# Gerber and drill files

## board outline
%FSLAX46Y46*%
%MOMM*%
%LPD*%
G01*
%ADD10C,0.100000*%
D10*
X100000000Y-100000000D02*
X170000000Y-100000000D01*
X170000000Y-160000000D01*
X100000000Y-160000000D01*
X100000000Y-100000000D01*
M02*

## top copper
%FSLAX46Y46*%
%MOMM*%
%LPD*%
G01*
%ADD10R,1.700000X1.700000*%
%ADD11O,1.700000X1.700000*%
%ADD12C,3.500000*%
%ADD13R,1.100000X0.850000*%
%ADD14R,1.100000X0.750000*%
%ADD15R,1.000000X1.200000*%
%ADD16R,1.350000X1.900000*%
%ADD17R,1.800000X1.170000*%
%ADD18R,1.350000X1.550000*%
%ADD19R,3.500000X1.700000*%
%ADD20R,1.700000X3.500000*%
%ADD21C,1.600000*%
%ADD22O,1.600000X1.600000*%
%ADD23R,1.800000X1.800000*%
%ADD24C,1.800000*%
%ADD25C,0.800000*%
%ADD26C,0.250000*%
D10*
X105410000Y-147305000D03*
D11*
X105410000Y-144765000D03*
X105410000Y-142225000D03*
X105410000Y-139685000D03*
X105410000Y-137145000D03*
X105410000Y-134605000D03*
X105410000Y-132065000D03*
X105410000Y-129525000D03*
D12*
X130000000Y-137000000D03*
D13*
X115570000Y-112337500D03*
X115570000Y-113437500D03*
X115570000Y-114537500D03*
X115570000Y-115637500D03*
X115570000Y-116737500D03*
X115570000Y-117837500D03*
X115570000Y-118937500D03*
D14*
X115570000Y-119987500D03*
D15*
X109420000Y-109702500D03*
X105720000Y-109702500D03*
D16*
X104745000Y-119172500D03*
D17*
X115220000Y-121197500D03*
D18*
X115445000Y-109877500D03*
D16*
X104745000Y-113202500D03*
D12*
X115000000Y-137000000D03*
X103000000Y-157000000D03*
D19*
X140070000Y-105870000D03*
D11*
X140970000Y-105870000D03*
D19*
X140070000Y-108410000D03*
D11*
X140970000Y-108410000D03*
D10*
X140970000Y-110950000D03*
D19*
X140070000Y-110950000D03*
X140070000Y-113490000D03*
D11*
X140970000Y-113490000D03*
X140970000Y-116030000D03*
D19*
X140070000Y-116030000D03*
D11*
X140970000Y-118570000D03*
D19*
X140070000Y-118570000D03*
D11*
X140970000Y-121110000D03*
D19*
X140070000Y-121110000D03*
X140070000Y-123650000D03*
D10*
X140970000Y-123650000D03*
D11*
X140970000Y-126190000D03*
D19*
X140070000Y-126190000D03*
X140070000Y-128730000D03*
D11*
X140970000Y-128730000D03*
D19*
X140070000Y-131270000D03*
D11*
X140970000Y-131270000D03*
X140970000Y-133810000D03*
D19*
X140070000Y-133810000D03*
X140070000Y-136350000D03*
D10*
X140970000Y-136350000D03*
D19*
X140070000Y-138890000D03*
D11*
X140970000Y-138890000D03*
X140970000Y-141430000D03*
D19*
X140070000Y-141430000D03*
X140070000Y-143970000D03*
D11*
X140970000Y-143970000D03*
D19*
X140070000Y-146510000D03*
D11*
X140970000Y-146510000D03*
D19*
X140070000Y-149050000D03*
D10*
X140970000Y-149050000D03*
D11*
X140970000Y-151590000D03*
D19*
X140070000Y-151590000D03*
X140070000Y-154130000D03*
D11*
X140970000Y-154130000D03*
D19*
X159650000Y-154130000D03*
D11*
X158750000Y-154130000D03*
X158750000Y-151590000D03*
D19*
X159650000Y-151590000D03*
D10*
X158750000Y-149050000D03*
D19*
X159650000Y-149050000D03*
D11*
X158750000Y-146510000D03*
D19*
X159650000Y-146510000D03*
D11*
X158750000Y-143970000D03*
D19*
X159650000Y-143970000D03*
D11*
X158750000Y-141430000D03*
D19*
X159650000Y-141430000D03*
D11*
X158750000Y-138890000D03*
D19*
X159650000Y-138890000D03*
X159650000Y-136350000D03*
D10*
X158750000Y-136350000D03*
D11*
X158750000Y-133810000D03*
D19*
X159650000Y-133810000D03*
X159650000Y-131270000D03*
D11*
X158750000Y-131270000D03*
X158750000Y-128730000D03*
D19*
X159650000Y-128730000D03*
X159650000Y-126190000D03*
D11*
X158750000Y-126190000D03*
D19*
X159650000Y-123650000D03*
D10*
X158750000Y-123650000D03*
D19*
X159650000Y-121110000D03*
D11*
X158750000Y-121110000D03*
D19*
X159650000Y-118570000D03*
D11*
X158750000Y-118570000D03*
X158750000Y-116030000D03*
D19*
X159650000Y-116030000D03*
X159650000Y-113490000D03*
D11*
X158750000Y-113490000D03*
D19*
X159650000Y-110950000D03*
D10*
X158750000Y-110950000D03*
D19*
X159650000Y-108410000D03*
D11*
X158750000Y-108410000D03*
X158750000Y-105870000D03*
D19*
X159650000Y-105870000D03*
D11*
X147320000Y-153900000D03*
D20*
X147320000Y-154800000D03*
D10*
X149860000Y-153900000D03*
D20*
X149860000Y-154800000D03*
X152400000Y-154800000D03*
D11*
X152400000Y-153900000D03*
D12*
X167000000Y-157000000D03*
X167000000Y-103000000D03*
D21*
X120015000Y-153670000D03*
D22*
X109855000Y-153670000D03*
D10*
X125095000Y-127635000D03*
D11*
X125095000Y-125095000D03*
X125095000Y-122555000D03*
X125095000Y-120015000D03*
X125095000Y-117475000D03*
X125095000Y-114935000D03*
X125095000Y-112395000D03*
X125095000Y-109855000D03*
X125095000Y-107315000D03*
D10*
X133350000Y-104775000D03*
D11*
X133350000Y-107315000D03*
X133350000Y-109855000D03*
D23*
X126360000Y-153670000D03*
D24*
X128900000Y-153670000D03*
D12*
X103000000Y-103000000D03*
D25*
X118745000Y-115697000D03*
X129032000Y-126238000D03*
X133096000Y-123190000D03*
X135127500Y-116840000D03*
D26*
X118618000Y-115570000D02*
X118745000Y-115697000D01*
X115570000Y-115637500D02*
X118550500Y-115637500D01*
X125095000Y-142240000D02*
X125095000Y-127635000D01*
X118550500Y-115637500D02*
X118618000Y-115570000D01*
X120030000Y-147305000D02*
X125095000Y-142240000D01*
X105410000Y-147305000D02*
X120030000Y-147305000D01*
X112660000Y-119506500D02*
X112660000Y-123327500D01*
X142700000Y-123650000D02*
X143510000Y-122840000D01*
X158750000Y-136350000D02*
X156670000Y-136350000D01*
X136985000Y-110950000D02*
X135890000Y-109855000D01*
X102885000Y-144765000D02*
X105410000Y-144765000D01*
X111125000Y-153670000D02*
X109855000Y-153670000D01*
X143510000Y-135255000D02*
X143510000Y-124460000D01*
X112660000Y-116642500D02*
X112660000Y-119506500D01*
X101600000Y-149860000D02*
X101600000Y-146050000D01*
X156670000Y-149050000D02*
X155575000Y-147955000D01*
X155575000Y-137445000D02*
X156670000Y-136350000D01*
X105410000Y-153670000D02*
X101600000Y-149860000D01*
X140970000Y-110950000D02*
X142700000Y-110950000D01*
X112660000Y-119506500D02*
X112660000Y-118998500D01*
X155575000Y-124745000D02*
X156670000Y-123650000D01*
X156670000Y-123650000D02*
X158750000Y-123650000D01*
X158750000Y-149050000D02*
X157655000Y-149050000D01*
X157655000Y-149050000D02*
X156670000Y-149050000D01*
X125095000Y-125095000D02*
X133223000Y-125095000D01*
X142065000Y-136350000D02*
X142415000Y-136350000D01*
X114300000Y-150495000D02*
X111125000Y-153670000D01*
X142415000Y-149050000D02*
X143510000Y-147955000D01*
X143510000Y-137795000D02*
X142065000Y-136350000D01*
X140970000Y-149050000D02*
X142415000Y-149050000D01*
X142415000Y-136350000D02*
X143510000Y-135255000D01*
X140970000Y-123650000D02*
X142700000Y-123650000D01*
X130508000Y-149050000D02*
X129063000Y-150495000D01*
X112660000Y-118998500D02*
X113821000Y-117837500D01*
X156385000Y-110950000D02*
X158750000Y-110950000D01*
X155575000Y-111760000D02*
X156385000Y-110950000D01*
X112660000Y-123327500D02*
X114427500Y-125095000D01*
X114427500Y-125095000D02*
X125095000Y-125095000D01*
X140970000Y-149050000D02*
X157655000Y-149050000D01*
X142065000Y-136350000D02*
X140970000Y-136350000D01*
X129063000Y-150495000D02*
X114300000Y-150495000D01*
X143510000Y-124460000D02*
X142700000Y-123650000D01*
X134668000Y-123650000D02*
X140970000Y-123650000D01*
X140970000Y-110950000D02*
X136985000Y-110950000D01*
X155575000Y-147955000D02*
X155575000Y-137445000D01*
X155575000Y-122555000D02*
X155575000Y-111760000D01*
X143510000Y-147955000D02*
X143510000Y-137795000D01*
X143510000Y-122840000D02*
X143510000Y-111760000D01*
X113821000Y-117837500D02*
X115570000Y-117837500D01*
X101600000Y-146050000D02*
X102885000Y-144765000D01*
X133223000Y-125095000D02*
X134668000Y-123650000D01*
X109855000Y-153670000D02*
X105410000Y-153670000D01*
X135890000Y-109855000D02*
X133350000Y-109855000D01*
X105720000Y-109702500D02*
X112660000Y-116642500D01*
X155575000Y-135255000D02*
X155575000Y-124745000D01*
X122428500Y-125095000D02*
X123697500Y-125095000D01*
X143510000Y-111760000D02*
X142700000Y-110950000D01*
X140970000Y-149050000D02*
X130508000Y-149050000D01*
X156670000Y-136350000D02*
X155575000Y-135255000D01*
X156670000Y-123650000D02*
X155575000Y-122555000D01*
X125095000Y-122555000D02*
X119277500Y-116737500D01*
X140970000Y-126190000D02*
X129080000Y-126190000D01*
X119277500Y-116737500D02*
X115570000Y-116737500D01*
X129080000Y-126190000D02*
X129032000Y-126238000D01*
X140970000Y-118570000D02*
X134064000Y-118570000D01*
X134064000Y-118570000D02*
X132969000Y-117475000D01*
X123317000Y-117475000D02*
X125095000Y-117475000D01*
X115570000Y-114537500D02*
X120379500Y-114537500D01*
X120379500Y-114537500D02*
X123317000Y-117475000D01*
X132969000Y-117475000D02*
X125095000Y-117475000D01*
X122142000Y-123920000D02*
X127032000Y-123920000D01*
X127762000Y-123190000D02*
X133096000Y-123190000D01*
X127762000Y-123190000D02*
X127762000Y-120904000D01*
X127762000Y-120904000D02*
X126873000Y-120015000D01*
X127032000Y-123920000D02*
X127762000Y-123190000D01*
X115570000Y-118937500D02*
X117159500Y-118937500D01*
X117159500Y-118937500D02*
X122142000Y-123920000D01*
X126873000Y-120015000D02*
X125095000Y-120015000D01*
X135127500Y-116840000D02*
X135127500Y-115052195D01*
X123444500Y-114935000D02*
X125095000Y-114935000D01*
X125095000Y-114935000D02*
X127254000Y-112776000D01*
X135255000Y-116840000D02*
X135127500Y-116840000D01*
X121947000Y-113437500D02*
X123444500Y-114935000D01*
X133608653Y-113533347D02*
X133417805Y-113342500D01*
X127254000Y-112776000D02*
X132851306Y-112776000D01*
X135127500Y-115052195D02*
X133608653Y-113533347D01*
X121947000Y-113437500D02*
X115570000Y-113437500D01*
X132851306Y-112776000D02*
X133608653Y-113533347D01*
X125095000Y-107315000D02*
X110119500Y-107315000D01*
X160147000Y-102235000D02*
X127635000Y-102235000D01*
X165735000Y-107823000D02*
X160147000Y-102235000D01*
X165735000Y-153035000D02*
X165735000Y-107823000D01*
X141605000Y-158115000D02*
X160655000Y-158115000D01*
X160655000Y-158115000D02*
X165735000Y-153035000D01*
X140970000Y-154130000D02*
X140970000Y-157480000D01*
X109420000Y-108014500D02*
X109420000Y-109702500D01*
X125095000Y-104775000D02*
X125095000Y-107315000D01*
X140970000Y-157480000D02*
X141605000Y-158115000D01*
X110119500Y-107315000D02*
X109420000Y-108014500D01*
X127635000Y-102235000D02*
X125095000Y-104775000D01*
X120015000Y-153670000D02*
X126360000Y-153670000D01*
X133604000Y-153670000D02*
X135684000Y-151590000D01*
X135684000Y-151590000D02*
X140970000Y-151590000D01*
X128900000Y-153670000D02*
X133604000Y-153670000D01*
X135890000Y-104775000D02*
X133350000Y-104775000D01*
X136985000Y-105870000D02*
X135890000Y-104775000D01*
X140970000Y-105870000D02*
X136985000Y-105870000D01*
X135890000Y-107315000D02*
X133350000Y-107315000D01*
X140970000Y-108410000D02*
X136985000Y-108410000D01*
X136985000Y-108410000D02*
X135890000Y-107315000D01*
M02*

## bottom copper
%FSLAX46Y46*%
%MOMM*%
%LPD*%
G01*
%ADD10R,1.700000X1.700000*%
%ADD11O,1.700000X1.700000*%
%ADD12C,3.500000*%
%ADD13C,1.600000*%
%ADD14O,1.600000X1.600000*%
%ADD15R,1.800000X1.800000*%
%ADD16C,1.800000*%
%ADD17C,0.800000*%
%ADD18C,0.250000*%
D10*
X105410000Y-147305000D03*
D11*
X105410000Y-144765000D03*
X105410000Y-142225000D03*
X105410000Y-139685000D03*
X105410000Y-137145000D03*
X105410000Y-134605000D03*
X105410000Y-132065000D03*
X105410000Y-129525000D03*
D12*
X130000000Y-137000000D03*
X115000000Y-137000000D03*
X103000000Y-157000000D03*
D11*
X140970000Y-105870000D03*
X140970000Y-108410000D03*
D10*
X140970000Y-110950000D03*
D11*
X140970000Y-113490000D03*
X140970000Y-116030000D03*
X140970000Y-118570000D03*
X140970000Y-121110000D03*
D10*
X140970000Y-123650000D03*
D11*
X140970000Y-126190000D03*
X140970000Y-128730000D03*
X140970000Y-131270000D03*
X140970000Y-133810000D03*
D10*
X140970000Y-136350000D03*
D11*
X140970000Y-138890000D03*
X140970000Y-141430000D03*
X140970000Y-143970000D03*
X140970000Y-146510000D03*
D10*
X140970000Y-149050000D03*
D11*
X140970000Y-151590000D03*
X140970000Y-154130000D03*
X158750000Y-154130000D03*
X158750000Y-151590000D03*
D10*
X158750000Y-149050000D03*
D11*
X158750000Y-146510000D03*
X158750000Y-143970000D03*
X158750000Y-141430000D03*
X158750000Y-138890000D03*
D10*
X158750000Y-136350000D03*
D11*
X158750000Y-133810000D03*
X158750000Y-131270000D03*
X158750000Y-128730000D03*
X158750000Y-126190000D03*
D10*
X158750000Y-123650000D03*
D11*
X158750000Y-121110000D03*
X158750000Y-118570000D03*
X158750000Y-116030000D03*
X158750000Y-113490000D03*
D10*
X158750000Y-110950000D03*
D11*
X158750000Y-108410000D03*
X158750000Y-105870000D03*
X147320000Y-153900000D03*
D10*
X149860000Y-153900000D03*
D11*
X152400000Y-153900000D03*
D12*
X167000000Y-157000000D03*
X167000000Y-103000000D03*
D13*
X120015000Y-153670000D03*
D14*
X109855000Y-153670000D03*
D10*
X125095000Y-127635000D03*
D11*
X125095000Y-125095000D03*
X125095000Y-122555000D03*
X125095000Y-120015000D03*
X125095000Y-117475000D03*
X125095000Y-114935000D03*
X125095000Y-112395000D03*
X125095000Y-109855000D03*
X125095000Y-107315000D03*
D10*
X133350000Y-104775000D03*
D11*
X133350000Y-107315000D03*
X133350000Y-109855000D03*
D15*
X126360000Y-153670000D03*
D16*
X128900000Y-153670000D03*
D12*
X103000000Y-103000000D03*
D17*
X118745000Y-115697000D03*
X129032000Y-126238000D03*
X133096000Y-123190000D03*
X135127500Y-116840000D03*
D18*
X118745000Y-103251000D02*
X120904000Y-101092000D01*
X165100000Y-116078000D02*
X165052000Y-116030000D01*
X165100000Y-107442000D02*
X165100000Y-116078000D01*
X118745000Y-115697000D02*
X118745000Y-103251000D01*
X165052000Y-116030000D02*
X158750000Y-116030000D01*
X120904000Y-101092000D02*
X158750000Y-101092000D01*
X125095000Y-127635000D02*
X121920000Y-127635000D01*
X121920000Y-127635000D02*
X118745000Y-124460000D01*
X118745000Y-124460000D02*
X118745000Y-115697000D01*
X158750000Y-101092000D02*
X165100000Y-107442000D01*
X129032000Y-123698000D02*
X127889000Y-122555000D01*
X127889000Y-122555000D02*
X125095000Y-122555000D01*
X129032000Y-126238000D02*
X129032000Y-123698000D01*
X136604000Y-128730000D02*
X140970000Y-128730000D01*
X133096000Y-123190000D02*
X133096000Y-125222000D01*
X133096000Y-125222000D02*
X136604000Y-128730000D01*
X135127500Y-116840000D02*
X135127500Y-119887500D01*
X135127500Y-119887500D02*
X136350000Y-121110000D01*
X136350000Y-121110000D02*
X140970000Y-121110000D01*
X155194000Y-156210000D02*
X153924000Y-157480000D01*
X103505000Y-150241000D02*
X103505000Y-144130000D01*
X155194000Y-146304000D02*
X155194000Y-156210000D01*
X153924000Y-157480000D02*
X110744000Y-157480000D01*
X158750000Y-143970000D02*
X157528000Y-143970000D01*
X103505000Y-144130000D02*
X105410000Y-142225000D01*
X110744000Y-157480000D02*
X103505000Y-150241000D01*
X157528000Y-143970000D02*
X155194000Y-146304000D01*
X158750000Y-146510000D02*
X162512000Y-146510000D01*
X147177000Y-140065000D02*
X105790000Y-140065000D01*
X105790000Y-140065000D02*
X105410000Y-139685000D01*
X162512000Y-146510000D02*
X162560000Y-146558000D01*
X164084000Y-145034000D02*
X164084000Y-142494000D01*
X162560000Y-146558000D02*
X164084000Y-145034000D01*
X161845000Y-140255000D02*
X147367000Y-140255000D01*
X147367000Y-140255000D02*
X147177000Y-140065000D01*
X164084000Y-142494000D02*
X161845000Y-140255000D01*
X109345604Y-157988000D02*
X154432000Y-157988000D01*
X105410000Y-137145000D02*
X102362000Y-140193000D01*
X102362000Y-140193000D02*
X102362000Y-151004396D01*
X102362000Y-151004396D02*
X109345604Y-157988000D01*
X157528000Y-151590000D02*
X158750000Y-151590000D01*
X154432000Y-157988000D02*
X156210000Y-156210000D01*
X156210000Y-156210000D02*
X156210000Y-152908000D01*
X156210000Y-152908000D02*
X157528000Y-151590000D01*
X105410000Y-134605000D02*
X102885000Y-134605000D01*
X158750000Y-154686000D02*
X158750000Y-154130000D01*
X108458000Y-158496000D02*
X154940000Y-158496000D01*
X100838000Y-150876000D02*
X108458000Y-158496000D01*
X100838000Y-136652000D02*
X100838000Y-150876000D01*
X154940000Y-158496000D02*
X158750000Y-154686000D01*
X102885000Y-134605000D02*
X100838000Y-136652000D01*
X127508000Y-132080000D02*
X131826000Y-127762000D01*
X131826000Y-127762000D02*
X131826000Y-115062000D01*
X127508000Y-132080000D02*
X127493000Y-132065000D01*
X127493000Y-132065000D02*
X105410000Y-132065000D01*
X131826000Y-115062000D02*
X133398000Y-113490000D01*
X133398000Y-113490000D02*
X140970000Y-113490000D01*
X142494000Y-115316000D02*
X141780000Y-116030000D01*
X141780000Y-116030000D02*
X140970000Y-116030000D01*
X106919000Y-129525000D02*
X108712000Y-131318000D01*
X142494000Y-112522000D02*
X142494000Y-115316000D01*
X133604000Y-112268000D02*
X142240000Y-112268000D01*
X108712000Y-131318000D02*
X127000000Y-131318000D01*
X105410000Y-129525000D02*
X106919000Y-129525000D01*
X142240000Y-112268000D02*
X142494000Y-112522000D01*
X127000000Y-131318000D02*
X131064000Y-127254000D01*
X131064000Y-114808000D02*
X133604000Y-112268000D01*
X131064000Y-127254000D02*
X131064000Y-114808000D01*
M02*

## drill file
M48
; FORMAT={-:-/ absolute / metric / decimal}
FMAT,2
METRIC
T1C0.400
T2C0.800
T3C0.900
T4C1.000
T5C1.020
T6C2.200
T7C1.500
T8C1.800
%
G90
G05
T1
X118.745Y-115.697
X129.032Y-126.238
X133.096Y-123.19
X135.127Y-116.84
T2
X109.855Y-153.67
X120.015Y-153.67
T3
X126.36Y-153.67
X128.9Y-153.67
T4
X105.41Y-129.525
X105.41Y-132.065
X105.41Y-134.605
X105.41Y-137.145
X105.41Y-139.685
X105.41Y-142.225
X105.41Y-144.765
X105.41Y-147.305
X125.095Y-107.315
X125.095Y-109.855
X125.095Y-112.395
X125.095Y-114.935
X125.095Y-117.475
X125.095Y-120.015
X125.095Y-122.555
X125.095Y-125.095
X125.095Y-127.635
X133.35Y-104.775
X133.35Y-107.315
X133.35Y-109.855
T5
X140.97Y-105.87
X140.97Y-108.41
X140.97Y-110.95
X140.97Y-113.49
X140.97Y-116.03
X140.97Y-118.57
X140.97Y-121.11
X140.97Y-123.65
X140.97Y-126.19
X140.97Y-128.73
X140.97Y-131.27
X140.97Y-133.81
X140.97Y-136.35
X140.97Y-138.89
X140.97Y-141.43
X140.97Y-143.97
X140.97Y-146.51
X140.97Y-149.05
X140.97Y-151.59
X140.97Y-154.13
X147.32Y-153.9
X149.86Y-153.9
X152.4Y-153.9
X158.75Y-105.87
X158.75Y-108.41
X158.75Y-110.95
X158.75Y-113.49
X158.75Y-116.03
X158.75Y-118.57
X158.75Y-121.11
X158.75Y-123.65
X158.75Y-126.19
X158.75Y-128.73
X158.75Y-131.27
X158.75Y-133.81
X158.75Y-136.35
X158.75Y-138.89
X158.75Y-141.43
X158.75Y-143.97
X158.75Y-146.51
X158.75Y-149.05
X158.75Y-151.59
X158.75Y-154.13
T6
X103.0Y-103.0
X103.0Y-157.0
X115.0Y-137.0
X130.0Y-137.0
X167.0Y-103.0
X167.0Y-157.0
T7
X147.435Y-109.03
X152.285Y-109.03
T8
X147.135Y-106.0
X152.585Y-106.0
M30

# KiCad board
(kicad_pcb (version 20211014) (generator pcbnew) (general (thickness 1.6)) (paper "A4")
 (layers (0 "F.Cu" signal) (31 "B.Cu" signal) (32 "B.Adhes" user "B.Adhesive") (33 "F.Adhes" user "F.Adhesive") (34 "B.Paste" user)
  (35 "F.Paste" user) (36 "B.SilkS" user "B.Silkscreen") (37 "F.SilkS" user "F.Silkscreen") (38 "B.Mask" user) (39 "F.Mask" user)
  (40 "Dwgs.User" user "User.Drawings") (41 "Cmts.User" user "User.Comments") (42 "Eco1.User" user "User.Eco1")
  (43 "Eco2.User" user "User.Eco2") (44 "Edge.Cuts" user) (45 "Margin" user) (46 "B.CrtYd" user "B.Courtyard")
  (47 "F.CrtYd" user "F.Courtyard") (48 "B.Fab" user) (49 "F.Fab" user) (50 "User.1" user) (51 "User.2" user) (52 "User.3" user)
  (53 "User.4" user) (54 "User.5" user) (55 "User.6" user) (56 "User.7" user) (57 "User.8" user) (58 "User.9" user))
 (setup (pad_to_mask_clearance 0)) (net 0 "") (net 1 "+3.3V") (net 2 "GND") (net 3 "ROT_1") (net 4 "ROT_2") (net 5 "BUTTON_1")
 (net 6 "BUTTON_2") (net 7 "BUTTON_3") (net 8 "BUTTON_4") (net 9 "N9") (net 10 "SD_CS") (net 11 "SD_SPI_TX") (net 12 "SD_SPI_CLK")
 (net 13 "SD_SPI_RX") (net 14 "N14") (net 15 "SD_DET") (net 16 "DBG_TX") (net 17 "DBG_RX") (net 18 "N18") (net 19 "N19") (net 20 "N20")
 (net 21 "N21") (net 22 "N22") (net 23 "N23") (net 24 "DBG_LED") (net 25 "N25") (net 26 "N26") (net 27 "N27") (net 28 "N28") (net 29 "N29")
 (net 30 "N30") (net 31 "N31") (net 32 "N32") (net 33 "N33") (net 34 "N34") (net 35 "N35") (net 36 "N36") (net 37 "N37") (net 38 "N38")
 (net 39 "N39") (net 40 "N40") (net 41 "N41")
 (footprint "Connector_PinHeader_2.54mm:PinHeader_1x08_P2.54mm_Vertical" (layer "F.Cu") (at 105.41 147.305 180)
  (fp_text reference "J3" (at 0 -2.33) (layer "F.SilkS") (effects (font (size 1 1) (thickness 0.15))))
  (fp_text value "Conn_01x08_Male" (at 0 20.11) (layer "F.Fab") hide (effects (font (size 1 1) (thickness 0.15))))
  (pad "1" thru_hole rect (at 0 0 180) (size 1.7 1.7) (drill 1) (layers *.Cu *.Mask) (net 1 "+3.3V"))
  (pad "2" thru_hole oval (at 0 2.54 180) (size 1.7 1.7) (drill 1) (layers *.Cu *.Mask) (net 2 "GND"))
  (pad "3" thru_hole oval (at 0 5.08 180) (size 1.7 1.7) (drill 1) (layers *.Cu *.Mask) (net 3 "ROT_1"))
  (pad "4" thru_hole oval (at 0 7.62 180) (size 1.7 1.7) (drill 1) (layers *.Cu *.Mask) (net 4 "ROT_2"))
  (pad "5" thru_hole oval (at 0 10.16 180) (size 1.7 1.7) (drill 1) (layers *.Cu *.Mask) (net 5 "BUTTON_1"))
  (pad "6" thru_hole oval (at 0 12.7 180) (size 1.7 1.7) (drill 1) (layers *.Cu *.Mask) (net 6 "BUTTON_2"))
  (pad "7" thru_hole oval (at 0 15.24 180) (size 1.7 1.7) (drill 1) (layers *.Cu *.Mask) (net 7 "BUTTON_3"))
  (pad "8" thru_hole oval (at 0 17.78 180) (size 1.7 1.7) (drill 1) (layers *.Cu *.Mask) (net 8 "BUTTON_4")))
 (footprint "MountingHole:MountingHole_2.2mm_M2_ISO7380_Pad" (layer "F.Cu") (at 130 137)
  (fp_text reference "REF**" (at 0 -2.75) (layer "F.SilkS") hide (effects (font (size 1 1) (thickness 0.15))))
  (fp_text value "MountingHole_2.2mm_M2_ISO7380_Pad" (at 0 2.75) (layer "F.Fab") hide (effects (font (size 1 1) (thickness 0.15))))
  (pad "1" thru_hole circle (at 0 0) (size 3.5 3.5) (drill 2.2) (layers *.Cu *.Mask)))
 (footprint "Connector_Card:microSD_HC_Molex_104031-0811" (layer "F.Cu") (at 110.12 115.4425 -90)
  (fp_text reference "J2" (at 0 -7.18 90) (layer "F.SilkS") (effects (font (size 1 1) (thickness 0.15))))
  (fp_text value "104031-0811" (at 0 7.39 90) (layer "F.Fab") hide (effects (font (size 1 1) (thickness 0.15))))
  (pad "1" smd rect (at -3.105 -5.45 270) (size 0.85 1.1) (layers "F.Cu" "F.Paste" "F.Mask") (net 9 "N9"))
  (pad "2" smd rect (at -2.005 -5.45 270) (size 0.85 1.1) (layers "F.Cu" "F.Paste" "F.Mask") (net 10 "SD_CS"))
  (pad "3" smd rect (at -0.905 -5.45 270) (size 0.85 1.1) (layers "F.Cu" "F.Paste" "F.Mask") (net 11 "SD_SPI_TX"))
  (pad "4" smd rect (at 0.195 -5.45 270) (size 0.85 1.1) (layers "F.Cu" "F.Paste" "F.Mask") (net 1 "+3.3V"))
  (pad "5" smd rect (at 1.295 -5.45 270) (size 0.85 1.1) (layers "F.Cu" "F.Paste" "F.Mask") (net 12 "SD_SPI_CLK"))
  (pad "6" smd rect (at 2.395 -5.45 270) (size 0.85 1.1) (layers "F.Cu" "F.Paste" "F.Mask") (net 2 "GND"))
  (pad "7" smd rect (at 3.495 -5.45 270) (size 0.85 1.1) (layers "F.Cu" "F.Paste" "F.Mask") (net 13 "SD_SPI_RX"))
  (pad "8" smd rect (at 4.545 -5.45 270) (size 0.75 1.1) (layers "F.Cu" "F.Paste" "F.Mask") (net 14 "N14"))
  (pad "9" smd rect (at -5.74 0.7 270) (size 1.2 1) (layers "F.Cu" "F.Paste" "F.Mask") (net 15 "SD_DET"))
  (pad "10" smd rect (at -5.74 4.4 270) (size 1.2 1) (layers "F.Cu" "F.Paste" "F.Mask") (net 2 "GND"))
  (pad "11" smd rect (at 3.73 5.375 270) (size 1.9 1.35) (layers "F.Cu" "F.Paste" "F.Mask"))
  (pad "11" smd rect (at 5.755 -5.1 270) (size 1.17 1.8) (layers "F.Cu" "F.Paste" "F.Mask"))
  (pad "11" smd rect (at -5.565 -5.325 270) (size 1.55 1.35) (layers "F.Cu" "F.Paste" "F.Mask"))
  (pad "11" smd rect (at -2.24 5.375 270) (size 1.9 1.35) (layers "F.Cu" "F.Paste" "F.Mask")))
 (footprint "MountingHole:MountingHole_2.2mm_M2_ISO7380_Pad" (layer "F.Cu") (at 115 137)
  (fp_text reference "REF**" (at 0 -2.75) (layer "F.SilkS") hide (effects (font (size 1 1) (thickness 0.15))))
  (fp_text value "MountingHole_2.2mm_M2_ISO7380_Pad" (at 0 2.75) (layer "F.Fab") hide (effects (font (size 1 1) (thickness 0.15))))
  (pad "1" thru_hole circle (at 0 0) (size 3.5 3.5) (drill 2.2) (layers *.Cu *.Mask)))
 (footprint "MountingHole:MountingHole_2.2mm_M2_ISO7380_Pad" (layer "F.Cu") (at 103 157)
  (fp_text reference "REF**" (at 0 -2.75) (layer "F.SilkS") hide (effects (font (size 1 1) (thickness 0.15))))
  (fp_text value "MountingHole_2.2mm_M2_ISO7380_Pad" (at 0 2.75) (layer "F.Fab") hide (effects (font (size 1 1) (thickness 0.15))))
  (pad "1" thru_hole circle (at 0 0) (size 3.5 3.5) (drill 2.2) (layers *.Cu *.Mask)))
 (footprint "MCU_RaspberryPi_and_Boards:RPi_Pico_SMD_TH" (layer "F.Cu") (at 149.86 130)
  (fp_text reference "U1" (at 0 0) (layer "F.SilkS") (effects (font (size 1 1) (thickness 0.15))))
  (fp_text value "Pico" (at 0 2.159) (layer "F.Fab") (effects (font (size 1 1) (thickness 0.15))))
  (pad "" np_thru_hole oval (at 2.425 -20.97) (size 1.5 1.5) (drill 1.5) (layers *.Cu *.Mask))
  (pad "" np_thru_hole oval (at -2.425 -20.97) (size 1.5 1.5) (drill 1.5) (layers *.Cu *.Mask))
  (pad "" np_thru_hole oval (at -2.725 -24) (size 1.8 1.8) (drill 1.8) (layers *.Cu *.Mask))
  (pad "" np_thru_hole oval (at 2.725 -24) (size 1.8 1.8) (drill 1.8) (layers *.Cu *.Mask))
  (pad "1" smd rect (at -8.89 -24.13) (size 3.5 1.7) (drill (offset -0.9 0)) (layers "F.Cu" "F.Mask") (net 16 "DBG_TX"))
  (pad "1" thru_hole oval (at -8.89 -24.13) (size 1.7 1.7) (drill 1.02) (layers *.Cu *.Mask) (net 16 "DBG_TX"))
  (pad "2" smd rect (at -8.89 -21.59) (size 3.5 1.7) (drill (offset -0.9 0)) (layers "F.Cu" "F.Mask") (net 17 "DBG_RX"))
  (pad "2" thru_hole oval (at -8.89 -21.59) (size 1.7 1.7) (drill 1.02) (layers *.Cu *.Mask) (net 17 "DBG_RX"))
  (pad "3" thru_hole rect (at -8.89 -19.05) (size 1.7 1.7) (drill 1.02) (layers *.Cu *.Mask) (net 2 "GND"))
  (pad "3" smd rect (at -8.89 -19.05) (size 3.5 1.7) (drill (offset -0.9 0)) (layers "F.Cu" "F.Mask") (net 2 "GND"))
  (pad "4" smd rect (at -8.89 -16.51) (size 3.5 1.7) (drill (offset -0.9 0)) (layers "F.Cu" "F.Mask") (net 7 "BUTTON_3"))
  (pad "4" thru_hole oval (at -8.89 -16.51) (size 1.7 1.7) (drill 1.02) (layers *.Cu *.Mask) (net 7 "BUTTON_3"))
  (pad "5" thru_hole oval (at -8.89 -13.97) (size 1.7 1.7) (drill 1.02) (layers *.Cu *.Mask) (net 8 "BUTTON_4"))
  (pad "5" smd rect (at -8.89 -13.97) (size 3.5 1.7) (drill (offset -0.9 0)) (layers "F.Cu" "F.Mask") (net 8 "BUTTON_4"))
  (pad "6" thru_hole oval (at -8.89 -11.43) (size 1.7 1.7) (drill 1.02) (layers *.Cu *.Mask) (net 11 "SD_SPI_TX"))
  (pad "6" smd rect (at -8.89 -11.43) (size 3.5 1.7) (drill (offset -0.9 0)) (layers "F.Cu" "F.Mask") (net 11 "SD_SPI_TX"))
  (pad "7" thru_hole oval (at -8.89 -8.89) (size 1.7 1.7) (drill 1.02) (layers *.Cu *.Mask) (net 10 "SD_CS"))
  (pad "7" smd rect (at -8.89 -8.89) (size 3.5 1.7) (drill (offset -0.9 0)) (layers "F.Cu" "F.Mask") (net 10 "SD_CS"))
  (pad "8" smd rect (at -8.89 -6.35) (size 3.5 1.7) (drill (offset -0.9 0)) (layers "F.Cu" "F.Mask") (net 2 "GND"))
  (pad "8" thru_hole rect (at -8.89 -6.35) (size 1.7 1.7) (drill 1.02) (layers *.Cu *.Mask) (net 2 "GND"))
  (pad "9" thru_hole oval (at -8.89 -3.81) (size 1.7 1.7) (drill 1.02) (layers *.Cu *.Mask) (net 12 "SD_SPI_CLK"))
  (pad "9" smd rect (at -8.89 -3.81) (size 3.5 1.7) (drill (offset -0.9 0)) (layers "F.Cu" "F.Mask") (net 12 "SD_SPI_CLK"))
  (pad "10" smd rect (at -8.89 -1.27) (size 3.5 1.7) (drill (offset -0.9 0)) (layers "F.Cu" "F.Mask") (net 13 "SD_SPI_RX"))
  (pad "10" thru_hole oval (at -8.89 -1.27) (size 1.7 1.7) (drill 1.02) (layers *.Cu *.Mask) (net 13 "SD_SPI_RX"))
  (pad "11" smd rect (at -8.89 1.27) (size 3.5 1.7) (drill (offset -0.9 0)) (layers "F.Cu" "F.Mask") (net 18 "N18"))
  (pad "11" thru_hole oval (at -8.89 1.27) (size 1.7 1.7) (drill 1.02) (layers *.Cu *.Mask) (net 18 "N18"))
  (pad "12" thru_hole oval (at -8.89 3.81) (size 1.7 1.7) (drill 1.02) (layers *.Cu *.Mask) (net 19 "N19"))
  (pad "12" smd rect (at -8.89 3.81) (size 3.5 1.7) (drill (offset -0.9 0)) (layers "F.Cu" "F.Mask") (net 19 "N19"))
  (pad "13" smd rect (at -8.89 6.35) (size 3.5 1.7) (drill (offset -0.9 0)) (layers "F.Cu" "F.Mask") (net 2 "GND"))
  (pad "13" thru_hole rect (at -8.89 6.35) (size 1.7 1.7) (drill 1.02) (layers *.Cu *.Mask) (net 2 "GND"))
  (pad "14" smd rect (at -8.89 8.89) (size 3.5 1.7) (drill (offset -0.9 0)) (layers "F.Cu" "F.Mask") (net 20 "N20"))
  (pad "14" thru_hole oval (at -8.89 8.89) (size 1.7 1.7) (drill 1.02) (layers *.Cu *.Mask) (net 20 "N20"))
  (pad "15" thru_hole oval (at -8.89 11.43) (size 1.7 1.7) (drill 1.02) (layers *.Cu *.Mask) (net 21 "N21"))
  (pad "15" smd rect (at -8.89 11.43) (size 3.5 1.7) (drill (offset -0.9 0)) (layers "F.Cu" "F.Mask") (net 21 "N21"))
  (pad "16" smd rect (at -8.89 13.97) (size 3.5 1.7) (drill (offset -0.9 0)) (layers "F.Cu" "F.Mask") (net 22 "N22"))
  (pad "16" thru_hole oval (at -8.89 13.97) (size 1.7 1.7) (drill 1.02) (layers *.Cu *.Mask) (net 22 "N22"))
  (pad "17" smd rect (at -8.89 16.51) (size 3.5 1.7) (drill (offset -0.9 0)) (layers "F.Cu" "F.Mask") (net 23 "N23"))
  (pad "17" thru_hole oval (at -8.89 16.51) (size 1.7 1.7) (drill 1.02) (layers *.Cu *.Mask) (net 23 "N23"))
  (pad "18" smd rect (at -8.89 19.05) (size 3.5 1.7) (drill (offset -0.9 0)) (layers "F.Cu" "F.Mask") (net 2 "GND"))
  (pad "18" thru_hole rect (at -8.89 19.05) (size 1.7 1.7) (drill 1.02) (layers *.Cu *.Mask) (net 2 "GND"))
  (pad "19" thru_hole oval (at -8.89 21.59) (size 1.7 1.7) (drill 1.02) (layers *.Cu *.Mask) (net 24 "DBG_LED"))
  (pad "19" smd rect (at -8.89 21.59) (size 3.5 1.7) (drill (offset -0.9 0)) (layers "F.Cu" "F.Mask") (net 24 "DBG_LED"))
  (pad "20" smd rect (at -8.89 24.13) (size 3.5 1.7) (drill (offset -0.9 0)) (layers "F.Cu" "F.Mask") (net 15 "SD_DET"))
  (pad "20" thru_hole oval (at -8.89 24.13) (size 1.7 1.7) (drill 1.02) (layers *.Cu *.Mask) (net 15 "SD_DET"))
  (pad "21" smd rect (at 8.89 24.13) (size 3.5 1.7) (drill (offset 0.9 0)) (layers "F.Cu" "F.Mask") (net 6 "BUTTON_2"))
  (pad "21" thru_hole oval (at 8.89 24.13) (size 1.7 1.7) (drill 1.02) (layers *.Cu *.Mask) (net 6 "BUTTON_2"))
  (pad "22" thru_hole oval (at 8.89 21.59) (size 1.7 1.7) (drill 1.02) (layers *.Cu *.Mask) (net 5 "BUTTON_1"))
  (pad "22" smd rect (at 8.89 21.59) (size 3.5 1.7) (drill (offset 0.9 0)) (layers "F.Cu" "F.Mask") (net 5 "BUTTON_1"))
  (pad "23" thru_hole rect (at 8.89 19.05) (size 1.7 1.7) (drill 1.02) (layers *.Cu *.Mask) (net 2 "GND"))
  (pad "23" smd rect (at 8.89 19.05) (size 3.5 1.7) (drill (offset 0.9 0)) (layers "F.Cu" "F.Mask") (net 2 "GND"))
  (pad "24" thru_hole oval (at 8.89 16.51) (size 1.7 1.7) (drill 1.02) (layers *.Cu *.Mask) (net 4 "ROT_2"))
  (pad "24" smd rect (at 8.89 16.51) (size 3.5 1.7) (drill (offset 0.9 0)) (layers "F.Cu" "F.Mask") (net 4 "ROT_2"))
  (pad "25" thru_hole oval (at 8.89 13.97) (size 1.7 1.7) (drill 1.02) (layers *.Cu *.Mask) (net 3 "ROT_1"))
  (pad "25" smd rect (at 8.89 13.97) (size 3.5 1.7) (drill (offset 0.9 0)) (layers "F.Cu" "F.Mask") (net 3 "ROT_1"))
  (pad "26" thru_hole oval (at 8.89 11.43) (size 1.7 1.7) (drill 1.02) (layers *.Cu *.Mask) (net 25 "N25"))
  (pad "26" smd rect (at 8.89 11.43) (size 3.5 1.7) (drill (offset 0.9 0)) (layers "F.Cu" "F.Mask") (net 25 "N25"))
  (pad "27" thru_hole oval (at 8.89 8.89) (size 1.7 1.7) (drill 1.02) (layers *.Cu *.Mask) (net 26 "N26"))
  (pad "27" smd rect (at 8.89 8.89) (size 3.5 1.7) (drill (offset 0.9 0)) (layers "F.Cu" "F.Mask") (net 26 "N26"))
  (pad "28" smd rect (at 8.89 6.35) (size 3.5 1.7) (drill (offset 0.9 0)) (layers "F.Cu" "F.Mask") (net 2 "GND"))
  (pad "28" thru_hole rect (at 8.89 6.35) (size 1.7 1.7) (drill 1.02) (layers *.Cu *.Mask) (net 2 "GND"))
  (pad "29" thru_hole oval (at 8.89 3.81) (size 1.7 1.7) (drill 1.02) (layers *.Cu *.Mask) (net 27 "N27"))
  (pad "29" smd rect (at 8.89 3.81) (size 3.5 1.7) (drill (offset 0.9 0)) (layers "F.Cu" "F.Mask") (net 27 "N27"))
  (pad "30" smd rect (at 8.89 1.27) (size 3.5 1.7) (drill (offset 0.9 0)) (layers "F.Cu" "F.Mask") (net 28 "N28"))
  (pad "30" thru_hole oval (at 8.89 1.27) (size 1.7 1.7) (drill 1.02) (layers *.Cu *.Mask) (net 28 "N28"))
  (pad "31" thru_hole oval (at 8.89 -1.27) (size 1.7 1.7) (drill 1.02) (layers *.Cu *.Mask) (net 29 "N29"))
  (pad "31" smd rect (at 8.89 -1.27) (size 3.5 1.7) (drill (offset 0.9 0)) (layers "F.Cu" "F.Mask") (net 29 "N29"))
  (pad "32" smd rect (at 8.89 -3.81) (size 3.5 1.7) (drill (offset 0.9 0)) (layers "F.Cu" "F.Mask") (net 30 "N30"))
  (pad "32" thru_hole oval (at 8.89 -3.81) (size 1.7 1.7) (drill 1.02) (layers *.Cu *.Mask) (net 30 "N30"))
  (pad "33" smd rect (at 8.89 -6.35) (size 3.5 1.7) (drill (offset 0.9 0)) (layers "F.Cu" "F.Mask") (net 2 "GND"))
  (pad "33" thru_hole rect (at 8.89 -6.35) (size 1.7 1.7) (drill 1.02) (layers *.Cu *.Mask) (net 2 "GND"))
  (pad "34" smd rect (at 8.89 -8.89) (size 3.5 1.7) (drill (offset 0.9 0)) (layers "F.Cu" "F.Mask") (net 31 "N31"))
  (pad "34" thru_hole oval (at 8.89 -8.89) (size 1.7 1.7) (drill 1.02) (layers *.Cu *.Mask) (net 31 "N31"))
  (pad "35" smd rect (at 8.89 -11.43) (size 3.5 1.7) (drill (offset 0.9 0)) (layers "F.Cu" "F.Mask") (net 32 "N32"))
  (pad "35" thru_hole oval (at 8.89 -11.43) (size 1.7 1.7) (drill 1.02) (layers *.Cu *.Mask) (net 32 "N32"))
  (pad "36" thru_hole oval (at 8.89 -13.97) (size 1.7 1.7) (drill 1.02) (layers *.Cu *.Mask) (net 1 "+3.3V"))
  (pad "36" smd rect (at 8.89 -13.97) (size 3.5 1.7) (drill (offset 0.9 0)) (layers "F.Cu" "F.Mask") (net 1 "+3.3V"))
  (pad "37" smd rect (at 8.89 -16.51) (size 3.5 1.7) (drill (offset 0.9 0)) (layers "F.Cu" "F.Mask") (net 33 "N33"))
  (pad "37" thru_hole oval (at 8.89 -16.51) (size 1.7 1.7) (drill 1.02) (layers *.Cu *.Mask) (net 33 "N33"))
  (pad "38" smd rect (at 8.89 -19.05) (size 3.5 1.7) (drill (offset 0.9 0)) (layers "F.Cu" "F.Mask") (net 2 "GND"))
  (pad "38" thru_hole rect (at 8.89 -19.05) (size 1.7 1.7) (drill 1.02) (layers *.Cu *.Mask) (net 2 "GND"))
  (pad "39" smd rect (at 8.89 -21.59) (size 3.5 1.7) (drill (offset 0.9 0)) (layers "F.Cu" "F.Mask") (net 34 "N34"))
  (pad "39" thru_hole oval (at 8.89 -21.59) (size 1.7 1.7) (drill 1.02) (layers *.Cu *.Mask) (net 34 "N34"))
  (pad "40" thru_hole oval (at 8.89 -24.13) (size 1.7 1.7) (drill 1.02) (layers *.Cu *.Mask) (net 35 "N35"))
  (pad "40" smd rect (at 8.89 -24.13) (size 3.5 1.7) (drill (offset 0.9 0)) (layers "F.Cu" "F.Mask") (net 35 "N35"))
  (pad "41" thru_hole oval (at -2.54 23.9) (size 1.7 1.7) (drill 1.02) (layers *.Cu *.Mask) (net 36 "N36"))
  (pad "41" smd rect (at -2.54 23.9 90) (size 3.5 1.7) (drill (offset -0.9 0)) (layers "F.Cu" "F.Mask") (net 36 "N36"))
  (pad "42" thru_hole rect (at 0 23.9) (size 1.7 1.7) (drill 1.02) (layers *.Cu *.Mask) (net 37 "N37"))
  (pad "42" smd rect (at 0 23.9 90) (size 3.5 1.7) (drill (offset -0.9 0)) (layers "F.Cu" "F.Mask") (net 37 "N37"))
  (pad "43" smd rect (at 2.54 23.9 90) (size 3.5 1.7) (drill (offset -0.9 0)) (layers "F.Cu" "F.Mask") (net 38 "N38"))
  (pad "43" thru_hole oval (at 2.54 23.9) (size 1.7 1.7) (drill 1.02) (layers *.Cu *.Mask) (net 38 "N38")))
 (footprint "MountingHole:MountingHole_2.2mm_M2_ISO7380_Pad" (layer "F.Cu") (at 167 157)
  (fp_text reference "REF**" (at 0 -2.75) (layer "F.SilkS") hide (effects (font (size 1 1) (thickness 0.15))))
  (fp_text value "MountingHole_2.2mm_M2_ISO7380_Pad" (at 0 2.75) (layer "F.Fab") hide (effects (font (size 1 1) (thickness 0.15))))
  (pad "1" thru_hole circle (at 0 0) (size 3.5 3.5) (drill 2.2) (layers *.Cu *.Mask)))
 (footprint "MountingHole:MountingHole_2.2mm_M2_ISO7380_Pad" (layer "F.Cu") (at 167 103)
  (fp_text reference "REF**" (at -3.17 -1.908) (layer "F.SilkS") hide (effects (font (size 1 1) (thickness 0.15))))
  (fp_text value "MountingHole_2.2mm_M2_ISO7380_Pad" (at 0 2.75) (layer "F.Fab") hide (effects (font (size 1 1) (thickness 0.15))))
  (pad "1" thru_hole circle (at 0 0) (size 3.5 3.5) (drill 2.2) (layers *.Cu *.Mask)))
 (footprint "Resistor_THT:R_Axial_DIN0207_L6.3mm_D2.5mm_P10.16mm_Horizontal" (layer "F.Cu") (at 120.015 153.67 180)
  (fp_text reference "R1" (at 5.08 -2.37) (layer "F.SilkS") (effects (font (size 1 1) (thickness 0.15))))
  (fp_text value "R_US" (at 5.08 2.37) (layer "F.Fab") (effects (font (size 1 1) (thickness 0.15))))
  (pad "1" thru_hole circle (at 0 0 180) (size 1.6 1.6) (drill 0.8) (layers *.Cu *.Mask) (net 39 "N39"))
  (pad "2" thru_hole oval (at 10.16 0 180) (size 1.6 1.6) (drill 0.8) (layers *.Cu *.Mask) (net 2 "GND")))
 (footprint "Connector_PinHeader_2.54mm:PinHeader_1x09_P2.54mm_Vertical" (layer "F.Cu") (at 125.095 127.635 180)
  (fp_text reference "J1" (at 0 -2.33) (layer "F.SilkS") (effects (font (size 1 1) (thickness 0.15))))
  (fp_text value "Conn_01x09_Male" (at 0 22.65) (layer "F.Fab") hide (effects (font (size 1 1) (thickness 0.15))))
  (pad "1" thru_hole rect (at 0 0 180) (size 1.7 1.7) (drill 1) (layers *.Cu *.Mask) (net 1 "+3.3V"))
  (pad "2" thru_hole oval (at 0 2.54 180) (size 1.7 1.7) (drill 1) (layers *.Cu *.Mask) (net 2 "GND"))
  (pad "3" thru_hole oval (at 0 5.08 180) (size 1.7 1.7) (drill 1) (layers *.Cu *.Mask) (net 12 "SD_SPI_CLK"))
  (pad "4" thru_hole oval (at 0 7.62 180) (size 1.7 1.7) (drill 1) (layers *.Cu *.Mask) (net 13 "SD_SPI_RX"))
  (pad "5" thru_hole oval (at 0 10.16 180) (size 1.7 1.7) (drill 1) (layers *.Cu *.Mask) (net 11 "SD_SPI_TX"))
  (pad "6" thru_hole oval (at 0 12.7 180) (size 1.7 1.7) (drill 1) (layers *.Cu *.Mask) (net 10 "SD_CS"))
  (pad "7" thru_hole oval (at 0 15.24 180) (size 1.7 1.7) (drill 1) (layers *.Cu *.Mask) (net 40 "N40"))
  (pad "8" thru_hole oval (at 0 17.78 180) (size 1.7 1.7) (drill 1) (layers *.Cu *.Mask) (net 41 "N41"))
  (pad "9" thru_hole oval (at 0 20.32 180) (size 1.7 1.7) (drill 1) (layers *.Cu *.Mask) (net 15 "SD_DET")))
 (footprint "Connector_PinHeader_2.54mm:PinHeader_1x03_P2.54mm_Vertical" (layer "F.Cu") (at 133.35 104.775)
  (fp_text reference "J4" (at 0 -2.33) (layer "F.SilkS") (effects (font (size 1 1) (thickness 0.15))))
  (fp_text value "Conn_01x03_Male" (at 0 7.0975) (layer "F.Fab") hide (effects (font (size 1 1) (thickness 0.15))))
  (pad "1" thru_hole rect (at 0 0) (size 1.7 1.7) (drill 1) (layers *.Cu *.Mask) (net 16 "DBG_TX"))
  (pad "2" thru_hole oval (at 0 2.54) (size 1.7 1.7) (drill 1) (layers *.Cu *.Mask) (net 17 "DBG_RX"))
  (pad "3" thru_hole oval (at 0 5.08) (size 1.7 1.7) (drill 1) (layers *.Cu *.Mask) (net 2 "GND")))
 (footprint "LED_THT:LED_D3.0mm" (layer "F.Cu") (at 126.36 153.67)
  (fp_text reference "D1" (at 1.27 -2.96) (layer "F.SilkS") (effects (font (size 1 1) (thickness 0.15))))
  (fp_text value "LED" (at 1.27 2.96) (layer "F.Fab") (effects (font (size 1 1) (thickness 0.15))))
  (pad "1" thru_hole rect (at 0 0) (size 1.8 1.8) (drill 0.9) (layers *.Cu *.Mask) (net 39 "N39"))
  (pad "2" thru_hole circle (at 2.54 0) (size 1.8 1.8) (drill 0.9) (layers *.Cu *.Mask) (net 24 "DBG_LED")))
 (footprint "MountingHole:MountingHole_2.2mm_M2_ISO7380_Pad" (layer "F.Cu") (at 103 103)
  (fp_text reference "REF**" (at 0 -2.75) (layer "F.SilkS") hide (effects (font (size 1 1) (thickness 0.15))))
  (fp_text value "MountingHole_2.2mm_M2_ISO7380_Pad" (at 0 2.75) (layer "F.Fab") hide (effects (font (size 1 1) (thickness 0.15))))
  (pad "1" thru_hole circle (at 0 0) (size 3.5 3.5) (drill 2.2) (layers *.Cu *.Mask)))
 (gr_rect (start 100 100) (end 170 160) (layer "Edge.Cuts") (width 0.1) (fill none))
 (segment (start 118.618 115.57) (end 118.745 115.697) (width 0.25) (layer "F.Cu") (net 1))
 (segment (start 115.57 115.6375) (end 118.5505 115.6375) (width 0.25) (layer "F.Cu") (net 1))
 (segment (start 125.095 142.24) (end 125.095 127.635) (width 0.25) (layer "F.Cu") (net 1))
 (segment (start 118.5505 115.6375) (end 118.618 115.57) (width 0.25) (layer "F.Cu") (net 1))
 (segment (start 120.03 147.305) (end 125.095 142.24) (width 0.25) (layer "F.Cu") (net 1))
 (segment (start 105.41 147.305) (end 120.03 147.305) (width 0.25) (layer "F.Cu") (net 1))
 (via (at 118.745 115.697) (size 0.8) (drill 0.4) (layers "F.Cu" "B.Cu") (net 1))
 (segment (start 118.745 103.251) (end 120.904 101.092) (width 0.25) (layer "B.Cu") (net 1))
 (segment (start 165.1 116.078) (end 165.052 116.03) (width 0.25) (layer "B.Cu") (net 1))
 (segment (start 165.1 107.442) (end 165.1 116.078) (width 0.25) (layer "B.Cu") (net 1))
 (segment (start 118.745 115.697) (end 118.745 103.251) (width 0.25) (layer "B.Cu") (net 1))
 (segment (start 165.052 116.03) (end 158.75 116.03) (width 0.25) (layer "B.Cu") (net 1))
 (segment (start 120.904 101.092) (end 158.75 101.092) (width 0.25) (layer "B.Cu") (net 1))
 (segment (start 125.095 127.635) (end 121.92 127.635) (width 0.25) (layer "B.Cu") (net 1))
 (segment (start 121.92 127.635) (end 118.745 124.46) (width 0.25) (layer "B.Cu") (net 1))
 (segment (start 118.745 124.46) (end 118.745 115.697) (width 0.25) (layer "B.Cu") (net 1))
 (segment (start 158.75 101.092) (end 165.1 107.442) (width 0.25) (layer "B.Cu") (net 1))
 (segment (start 112.66 119.5065) (end 112.66 123.3275) (width 0.25) (layer "F.Cu") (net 2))
 (segment (start 142.7 123.65) (end 143.51 122.84) (width 0.25) (layer "F.Cu") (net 2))
 (segment (start 158.75 136.35) (end 156.67 136.35) (width 0.25) (layer "F.Cu") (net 2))
 (segment (start 136.985 110.95) (end 135.89 109.855) (width 0.25) (layer "F.Cu") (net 2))
 (segment (start 102.885 144.765) (end 105.41 144.765) (width 0.25) (layer "F.Cu") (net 2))
 (segment (start 111.125 153.67) (end 109.855 153.67) (width 0.25) (layer "F.Cu") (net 2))
 (segment (start 143.51 135.255) (end 143.51 124.46) (width 0.25) (layer "F.Cu") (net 2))
 (segment (start 112.66 116.6425) (end 112.66 119.5065) (width 0.25) (layer "F.Cu") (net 2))
 (segment (start 101.6 149.86) (end 101.6 146.05) (width 0.25) (layer "F.Cu") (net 2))
 (segment (start 156.67 149.05) (end 155.575 147.955) (width 0.25) (layer "F.Cu") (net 2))
 (segment (start 155.575 137.445) (end 156.67 136.35) (width 0.25) (layer "F.Cu") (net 2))
 (segment (start 105.41 153.67) (end 101.6 149.86) (width 0.25) (layer "F.Cu") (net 2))
 (segment (start 140.97 110.95) (end 142.7 110.95) (width 0.25) (layer "F.Cu") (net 2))
 (segment (start 112.66 119.5065) (end 112.66 118.9985) (width 0.25) (layer "F.Cu") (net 2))
 (segment (start 155.575 124.745) (end 156.67 123.65) (width 0.25) (layer "F.Cu") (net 2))
 (segment (start 156.67 123.65) (end 158.75 123.65) (width 0.25) (layer "F.Cu") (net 2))
 (segment (start 158.75 149.05) (end 157.655 149.05) (width 0.25) (layer "F.Cu") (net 2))
 (segment (start 157.655 149.05) (end 156.67 149.05) (width 0.25) (layer "F.Cu") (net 2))
 (segment (start 125.095 125.095) (end 133.223 125.095) (width 0.25) (layer "F.Cu") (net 2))
 (segment (start 142.065 136.35) (end 142.415 136.35) (width 0.25) (layer "F.Cu") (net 2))
 (segment (start 114.3 150.495) (end 111.125 153.67) (width 0.25) (layer "F.Cu") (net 2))
 (segment (start 142.415 149.05) (end 143.51 147.955) (width 0.25) (layer "F.Cu") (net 2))
 (segment (start 143.51 137.795) (end 142.065 136.35) (width 0.25) (layer "F.Cu") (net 2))
 (segment (start 140.97 149.05) (end 142.415 149.05) (width 0.25) (layer "F.Cu") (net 2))
 (segment (start 142.415 136.35) (end 143.51 135.255) (width 0.25) (layer "F.Cu") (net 2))
 (segment (start 140.97 123.65) (end 142.7 123.65) (width 0.25) (layer "F.Cu") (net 2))
 (segment (start 130.508 149.05) (end 129.063 150.495) (width 0.25) (layer "F.Cu") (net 2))
 (segment (start 112.66 118.9985) (end 113.821 117.8375) (width 0.25) (layer "F.Cu") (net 2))
 (segment (start 156.385 110.95) (end 158.75 110.95) (width 0.25) (layer "F.Cu") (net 2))
 (segment (start 155.575 111.76) (end 156.385 110.95) (width 0.25) (layer "F.Cu") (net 2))
 (segment (start 112.66 123.3275) (end 114.4275 125.095) (width 0.25) (layer "F.Cu") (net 2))
 (segment (start 114.4275 125.095) (end 125.095 125.095) (width 0.25) (layer "F.Cu") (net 2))
 (segment (start 140.97 149.05) (end 157.655 149.05) (width 0.25) (layer "F.Cu") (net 2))
 (segment (start 142.065 136.35) (end 140.97 136.35) (width 0.25) (layer "F.Cu") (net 2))
 (segment (start 129.063 150.495) (end 114.3 150.495) (width 0.25) (layer "F.Cu") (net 2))
 (segment (start 143.51 124.46) (end 142.7 123.65) (width 0.25) (layer "F.Cu") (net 2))
 (segment (start 134.668 123.65) (end 140.97 123.65) (width 0.25) (layer "F.Cu") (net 2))
 (segment (start 140.97 110.95) (end 136.985 110.95) (width 0.25) (layer "F.Cu") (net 2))
 (segment (start 155.575 147.955) (end 155.575 137.445) (width 0.25) (layer "F.Cu") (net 2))
 (segment (start 155.575 122.555) (end 155.575 111.76) (width 0.25) (layer "F.Cu") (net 2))
 (segment (start 143.51 147.955) (end 143.51 137.795) (width 0.25) (layer "F.Cu") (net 2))
 (segment (start 143.51 122.84) (end 143.51 111.76) (width 0.25) (layer "F.Cu") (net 2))
 (segment (start 113.821 117.8375) (end 115.57 117.8375) (width 0.25) (layer "F.Cu") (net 2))
 (segment (start 101.6 146.05) (end 102.885 144.765) (width 0.25) (layer "F.Cu") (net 2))
 (segment (start 133.223 125.095) (end 134.668 123.65) (width 0.25) (layer "F.Cu") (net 2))
 (segment (start 109.855 153.67) (end 105.41 153.67) (width 0.25) (layer "F.Cu") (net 2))
 (segment (start 135.89 109.855) (end 133.35 109.855) (width 0.25) (layer "F.Cu") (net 2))
 (segment (start 105.72 109.7025) (end 112.66 116.6425) (width 0.25) (layer "F.Cu") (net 2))
 (segment (start 155.575 135.255) (end 155.575 124.745) (width 0.25) (layer "F.Cu") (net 2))
 (segment (start 122.4285 125.095) (end 123.6975 125.095) (width 0.25) (layer "F.Cu") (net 2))
 (segment (start 143.51 111.76) (end 142.7 110.95) (width 0.25) (layer "F.Cu") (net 2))
 (segment (start 140.97 149.05) (end 130.508 149.05) (width 0.25) (layer "F.Cu") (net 2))
 (segment (start 156.67 136.35) (end 155.575 135.255) (width 0.25) (layer "F.Cu") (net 2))
 (segment (start 156.67 123.65) (end 155.575 122.555) (width 0.25) (layer "F.Cu") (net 2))
 (segment (start 125.095 122.555) (end 119.2775 116.7375) (width 0.25) (layer "F.Cu") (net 12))
 (segment (start 140.97 126.19) (end 129.08 126.19) (width 0.25) (layer "F.Cu") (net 12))
 (segment (start 119.2775 116.7375) (end 115.57 116.7375) (width 0.25) (layer "F.Cu") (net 12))
 (segment (start 129.08 126.19) (end 129.032 126.238) (width 0.25) (layer "F.Cu") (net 12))
 (via (at 129.032 126.238) (size 0.8) (drill 0.4) (layers "F.Cu" "B.Cu") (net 12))
 (segment (start 129.032 123.698) (end 127.889 122.555) (width 0.25) (layer "B.Cu") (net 12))
 (segment (start 127.889 122.555) (end 125.095 122.555) (width 0.25) (layer "B.Cu") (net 12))
 (segment (start 129.032 126.238) (end 129.032 123.698) (width 0.25) (layer "B.Cu") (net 12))
 (segment (start 140.97 118.57) (end 134.064 118.57) (width 0.25) (layer "F.Cu") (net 11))
 (segment (start 134.064 118.57) (end 132.969 117.475) (width 0.25) (layer "F.Cu") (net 11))
 (segment (start 123.317 117.475) (end 125.095 117.475) (width 0.25) (layer "F.Cu") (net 11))
 (segment (start 115.57 114.5375) (end 120.3795 114.5375) (width 0.25) (layer "F.Cu") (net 11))
 (segment (start 120.3795 114.5375) (end 123.317 117.475) (width 0.25) (layer "F.Cu") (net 11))
 (segment (start 132.969 117.475) (end 125.095 117.475) (width 0.25) (layer "F.Cu") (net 11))
 (segment (start 122.142 123.92) (end 127.032 123.92) (width 0.25) (layer "F.Cu") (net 13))
 (segment (start 127.762 123.19) (end 133.096 123.19) (width 0.25) (layer "F.Cu") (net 13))
 (segment (start 127.762 123.19) (end 127.762 120.904) (width 0.25) (layer "F.Cu") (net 13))
 (segment (start 127.762 120.904) (end 126.873 120.015) (width 0.25) (layer "F.Cu") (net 13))
 (segment (start 127.032 123.92) (end 127.762 123.19) (width 0.25) (layer "F.Cu") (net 13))
 (segment (start 115.57 118.9375) (end 117.1595 118.9375) (width 0.25) (layer "F.Cu") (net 13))
 (segment (start 117.1595 118.9375) (end 122.142 123.92) (width 0.25) (layer "F.Cu") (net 13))
 (segment (start 126.873 120.015) (end 125.095 120.015) (width 0.25) (layer "F.Cu") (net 13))
 (via (at 133.096 123.19) (size 0.8) (drill 0.4) (layers "F.Cu" "B.Cu") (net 13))
 (segment (start 136.604 128.73) (end 140.97 128.73) (width 0.25) (layer "B.Cu") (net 13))
 (segment (start 133.096 123.19) (end 133.096 125.222) (width 0.25) (layer "B.Cu") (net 13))
 (segment (start 133.096 125.222) (end 136.604 128.73) (width 0.25) (layer "B.Cu") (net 13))
 (segment (start 135.1275 116.84) (end 135.1275 115.052195) (width 0.25) (layer "F.Cu") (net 10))
 (segment (start 123.4445 114.935) (end 125.095 114.935) (width 0.25) (layer "F.Cu") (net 10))
 (segment (start 125.095 114.935) (end 127.254 112.776) (width 0.25) (layer "F.Cu") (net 10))
 (segment (start 135.255 116.84) (end 135.1275 116.84) (width 0.25) (layer "F.Cu") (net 10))
 (segment (start 121.947 113.4375) (end 123.4445 114.935) (width 0.25) (layer "F.Cu") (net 10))
 (segment (start 133.608653 113.533347) (end 133.417805 113.3425) (width 0.25) (layer "F.Cu") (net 10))
 (segment (start 127.254 112.776) (end 132.851306 112.776) (width 0.25) (layer "F.Cu") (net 10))
 (segment (start 135.1275 115.052195) (end 133.608653 113.533347) (width 0.25) (layer "F.Cu") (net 10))
 (segment (start 121.947 113.4375) (end 115.57 113.4375) (width 0.25) (layer "F.Cu") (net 10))
 (segment (start 132.851306 112.776) (end 133.608653 113.533347) (width 0.25) (layer "F.Cu") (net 10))
 (via (at 135.1275 116.84) (size 0.8) (drill 0.4) (layers "F.Cu" "B.Cu") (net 10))
 (segment (start 135.1275 116.84) (end 135.1275 119.8875) (width 0.25) (layer "B.Cu") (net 10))
 (segment (start 135.1275 119.8875) (end 136.35 121.11) (width 0.25) (layer "B.Cu") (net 10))
 (segment (start 136.35 121.11) (end 140.97 121.11) (width 0.25) (layer "B.Cu") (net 10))
 (segment (start 125.095 107.315) (end 110.1195 107.315) (width 0.25) (layer "F.Cu") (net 15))
 (segment (start 160.147 102.235) (end 127.635 102.235) (width 0.25) (layer "F.Cu") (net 15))
 (segment (start 165.735 107.823) (end 160.147 102.235) (width 0.25) (layer "F.Cu") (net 15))
 (segment (start 165.735 153.035) (end 165.735 107.823) (width 0.25) (layer "F.Cu") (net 15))
 (segment (start 141.605 158.115) (end 160.655 158.115) (width 0.25) (layer "F.Cu") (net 15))
 (segment (start 160.655 158.115) (end 165.735 153.035) (width 0.25) (layer "F.Cu") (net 15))
 (segment (start 140.97 154.13) (end 140.97 157.48) (width 0.25) (layer "F.Cu") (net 15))
 (segment (start 109.42 108.0145) (end 109.42 109.7025) (width 0.25) (layer "F.Cu") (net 15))
 (segment (start 125.095 104.775) (end 125.095 107.315) (width 0.25) (layer "F.Cu") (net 15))
 (segment (start 140.97 157.48) (end 141.605 158.115) (width 0.25) (layer "F.Cu") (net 15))
 (segment (start 110.1195 107.315) (end 109.42 108.0145) (width 0.25) (layer "F.Cu") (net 15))
 (segment (start 127.635 102.235) (end 125.095 104.775) (width 0.25) (layer "F.Cu") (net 15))
 (segment (start 120.015 153.67) (end 126.36 153.67) (width 0.25) (layer "F.Cu") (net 39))
 (segment (start 133.604 153.67) (end 135.684 151.59) (width 0.25) (layer "F.Cu") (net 24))
 (segment (start 135.684 151.59) (end 140.97 151.59) (width 0.25) (layer "F.Cu") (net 24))
 (segment (start 128.9 153.67) (end 133.604 153.67) (width 0.25) (layer "F.Cu") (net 24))
 (segment (start 155.194 156.21) (end 153.924 157.48) (width 0.25) (layer "B.Cu") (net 3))
 (segment (start 103.505 150.241) (end 103.505 144.13) (width 0.25) (layer "B.Cu") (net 3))
 (segment (start 155.194 146.304) (end 155.194 156.21) (width 0.25) (layer "B.Cu") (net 3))
 (segment (start 153.924 157.48) (end 110.744 157.48) (width 0.25) (layer "B.Cu") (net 3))
 (segment (start 158.75 143.97) (end 157.528 143.97) (width 0.25) (layer "B.Cu") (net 3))
 (segment (start 103.505 144.13) (end 105.41 142.225) (width 0.25) (layer "B.Cu") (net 3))
 (segment (start 110.744 157.48) (end 103.505 150.241) (width 0.25) (layer "B.Cu") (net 3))
 (segment (start 157.528 143.97) (end 155.194 146.304) (width 0.25) (layer "B.Cu") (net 3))
 (segment (start 158.75 146.51) (end 162.512 146.51) (width 0.25) (layer "B.Cu") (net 4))
 (segment (start 147.177 140.065) (end 105.79 140.065) (width 0.25) (layer "B.Cu") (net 4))
 (segment (start 105.79 140.065) (end 105.41 139.685) (width 0.25) (layer "B.Cu") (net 4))
 (segment (start 162.512 146.51) (end 162.56 146.558) (width 0.25) (layer "B.Cu") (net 4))
 (segment (start 164.084 145.034) (end 164.084 142.494) (width 0.25) (layer "B.Cu") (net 4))
 (segment (start 162.56 146.558) (end 164.084 145.034) (width 0.25) (layer "B.Cu") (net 4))
 (segment (start 161.845 140.255) (end 147.367 140.255) (width 0.25) (layer "B.Cu") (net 4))
 (segment (start 147.367 140.255) (end 147.177 140.065) (width 0.25) (layer "B.Cu") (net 4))
 (segment (start 164.084 142.494) (end 161.845 140.255) (width 0.25) (layer "B.Cu") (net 4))
 (segment (start 109.345604 157.988) (end 154.432 157.988) (width 0.25) (layer "B.Cu") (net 5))
 (segment (start 105.41 137.145) (end 102.362 140.193) (width 0.25) (layer "B.Cu") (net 5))
 (segment (start 102.362 140.193) (end 102.362 151.004396) (width 0.25) (layer "B.Cu") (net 5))
 (segment (start 102.362 151.004396) (end 109.345604 157.988) (width 0.25) (layer "B.Cu") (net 5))
 (segment (start 157.528 151.59) (end 158.75 151.59) (width 0.25) (layer "B.Cu") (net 5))
 (segment (start 154.432 157.988) (end 156.21 156.21) (width 0.25) (layer "B.Cu") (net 5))
 (segment (start 156.21 156.21) (end 156.21 152.908) (width 0.25) (layer "B.Cu") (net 5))
 (segment (start 156.21 152.908) (end 157.528 151.59) (width 0.25) (layer "B.Cu") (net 5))
 (segment (start 105.41 134.605) (end 102.885 134.605) (width 0.25) (layer "B.Cu") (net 6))
 (segment (start 158.75 154.686) (end 158.75 154.13) (width 0.25) (layer "B.Cu") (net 6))
 (segment (start 108.458 158.496) (end 154.94 158.496) (width 0.25) (layer "B.Cu") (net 6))
 (segment (start 100.838 150.876) (end 108.458 158.496) (width 0.25) (layer "B.Cu") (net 6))
 (segment (start 100.838 136.652) (end 100.838 150.876) (width 0.25) (layer "B.Cu") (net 6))
 (segment (start 154.94 158.496) (end 158.75 154.686) (width 0.25) (layer "B.Cu") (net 6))
 (segment (start 102.885 134.605) (end 100.838 136.652) (width 0.25) (layer "B.Cu") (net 6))
 (segment (start 127.508 132.08) (end 131.826 127.762) (width 0.25) (layer "B.Cu") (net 7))
 (segment (start 131.826 127.762) (end 131.826 115.062) (width 0.25) (layer "B.Cu") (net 7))
 (segment (start 127.508 132.08) (end 127.493 132.065) (width 0.25) (layer "B.Cu") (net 7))
 (segment (start 127.493 132.065) (end 105.41 132.065) (width 0.25) (layer "B.Cu") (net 7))
 (segment (start 131.826 115.062) (end 133.398 113.49) (width 0.25) (layer "B.Cu") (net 7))
 (segment (start 133.398 113.49) (end 140.97 113.49) (width 0.25) (layer "B.Cu") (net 7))
 (segment (start 142.494 115.316) (end 141.78 116.03) (width 0.25) (layer "B.Cu") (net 8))
 (segment (start 141.78 116.03) (end 140.97 116.03) (width 0.25) (layer "B.Cu") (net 8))
 (segment (start 106.919 129.525) (end 108.712 131.318) (width 0.25) (layer "B.Cu") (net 8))
 (segment (start 142.494 112.522) (end 142.494 115.316) (width 0.25) (layer "B.Cu") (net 8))
 (segment (start 133.604 112.268) (end 142.24 112.268) (width 0.25) (layer "B.Cu") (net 8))
 (segment (start 108.712 131.318) (end 127 131.318) (width 0.25) (layer "B.Cu") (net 8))
 (segment (start 105.41 129.525) (end 106.919 129.525) (width 0.25) (layer "B.Cu") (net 8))
 (segment (start 142.24 112.268) (end 142.494 112.522) (width 0.25) (layer "B.Cu") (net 8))
 (segment (start 127 131.318) (end 131.064 127.254) (width 0.25) (layer "B.Cu") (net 8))
 (segment (start 131.064 114.808) (end 133.604 112.268) (width 0.25) (layer "B.Cu") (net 8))
 (segment (start 131.064 127.254) (end 131.064 114.808) (width 0.25) (layer "B.Cu") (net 8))
 (segment (start 135.89 104.775) (end 133.35 104.775) (width 0.25) (layer "F.Cu") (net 16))
 (segment (start 136.985 105.87) (end 135.89 104.775) (width 0.25) (layer "F.Cu") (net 16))
 (segment (start 140.97 105.87) (end 136.985 105.87) (width 0.25) (layer "F.Cu") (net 16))
 (segment (start 135.89 107.315) (end 133.35 107.315) (width 0.25) (layer "F.Cu") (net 17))
 (segment (start 140.97 108.41) (end 136.985 108.41) (width 0.25) (layer "F.Cu") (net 17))
 (segment (start 136.985 108.41) (end 135.89 107.315) (width 0.25) (layer "F.Cu") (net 17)))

